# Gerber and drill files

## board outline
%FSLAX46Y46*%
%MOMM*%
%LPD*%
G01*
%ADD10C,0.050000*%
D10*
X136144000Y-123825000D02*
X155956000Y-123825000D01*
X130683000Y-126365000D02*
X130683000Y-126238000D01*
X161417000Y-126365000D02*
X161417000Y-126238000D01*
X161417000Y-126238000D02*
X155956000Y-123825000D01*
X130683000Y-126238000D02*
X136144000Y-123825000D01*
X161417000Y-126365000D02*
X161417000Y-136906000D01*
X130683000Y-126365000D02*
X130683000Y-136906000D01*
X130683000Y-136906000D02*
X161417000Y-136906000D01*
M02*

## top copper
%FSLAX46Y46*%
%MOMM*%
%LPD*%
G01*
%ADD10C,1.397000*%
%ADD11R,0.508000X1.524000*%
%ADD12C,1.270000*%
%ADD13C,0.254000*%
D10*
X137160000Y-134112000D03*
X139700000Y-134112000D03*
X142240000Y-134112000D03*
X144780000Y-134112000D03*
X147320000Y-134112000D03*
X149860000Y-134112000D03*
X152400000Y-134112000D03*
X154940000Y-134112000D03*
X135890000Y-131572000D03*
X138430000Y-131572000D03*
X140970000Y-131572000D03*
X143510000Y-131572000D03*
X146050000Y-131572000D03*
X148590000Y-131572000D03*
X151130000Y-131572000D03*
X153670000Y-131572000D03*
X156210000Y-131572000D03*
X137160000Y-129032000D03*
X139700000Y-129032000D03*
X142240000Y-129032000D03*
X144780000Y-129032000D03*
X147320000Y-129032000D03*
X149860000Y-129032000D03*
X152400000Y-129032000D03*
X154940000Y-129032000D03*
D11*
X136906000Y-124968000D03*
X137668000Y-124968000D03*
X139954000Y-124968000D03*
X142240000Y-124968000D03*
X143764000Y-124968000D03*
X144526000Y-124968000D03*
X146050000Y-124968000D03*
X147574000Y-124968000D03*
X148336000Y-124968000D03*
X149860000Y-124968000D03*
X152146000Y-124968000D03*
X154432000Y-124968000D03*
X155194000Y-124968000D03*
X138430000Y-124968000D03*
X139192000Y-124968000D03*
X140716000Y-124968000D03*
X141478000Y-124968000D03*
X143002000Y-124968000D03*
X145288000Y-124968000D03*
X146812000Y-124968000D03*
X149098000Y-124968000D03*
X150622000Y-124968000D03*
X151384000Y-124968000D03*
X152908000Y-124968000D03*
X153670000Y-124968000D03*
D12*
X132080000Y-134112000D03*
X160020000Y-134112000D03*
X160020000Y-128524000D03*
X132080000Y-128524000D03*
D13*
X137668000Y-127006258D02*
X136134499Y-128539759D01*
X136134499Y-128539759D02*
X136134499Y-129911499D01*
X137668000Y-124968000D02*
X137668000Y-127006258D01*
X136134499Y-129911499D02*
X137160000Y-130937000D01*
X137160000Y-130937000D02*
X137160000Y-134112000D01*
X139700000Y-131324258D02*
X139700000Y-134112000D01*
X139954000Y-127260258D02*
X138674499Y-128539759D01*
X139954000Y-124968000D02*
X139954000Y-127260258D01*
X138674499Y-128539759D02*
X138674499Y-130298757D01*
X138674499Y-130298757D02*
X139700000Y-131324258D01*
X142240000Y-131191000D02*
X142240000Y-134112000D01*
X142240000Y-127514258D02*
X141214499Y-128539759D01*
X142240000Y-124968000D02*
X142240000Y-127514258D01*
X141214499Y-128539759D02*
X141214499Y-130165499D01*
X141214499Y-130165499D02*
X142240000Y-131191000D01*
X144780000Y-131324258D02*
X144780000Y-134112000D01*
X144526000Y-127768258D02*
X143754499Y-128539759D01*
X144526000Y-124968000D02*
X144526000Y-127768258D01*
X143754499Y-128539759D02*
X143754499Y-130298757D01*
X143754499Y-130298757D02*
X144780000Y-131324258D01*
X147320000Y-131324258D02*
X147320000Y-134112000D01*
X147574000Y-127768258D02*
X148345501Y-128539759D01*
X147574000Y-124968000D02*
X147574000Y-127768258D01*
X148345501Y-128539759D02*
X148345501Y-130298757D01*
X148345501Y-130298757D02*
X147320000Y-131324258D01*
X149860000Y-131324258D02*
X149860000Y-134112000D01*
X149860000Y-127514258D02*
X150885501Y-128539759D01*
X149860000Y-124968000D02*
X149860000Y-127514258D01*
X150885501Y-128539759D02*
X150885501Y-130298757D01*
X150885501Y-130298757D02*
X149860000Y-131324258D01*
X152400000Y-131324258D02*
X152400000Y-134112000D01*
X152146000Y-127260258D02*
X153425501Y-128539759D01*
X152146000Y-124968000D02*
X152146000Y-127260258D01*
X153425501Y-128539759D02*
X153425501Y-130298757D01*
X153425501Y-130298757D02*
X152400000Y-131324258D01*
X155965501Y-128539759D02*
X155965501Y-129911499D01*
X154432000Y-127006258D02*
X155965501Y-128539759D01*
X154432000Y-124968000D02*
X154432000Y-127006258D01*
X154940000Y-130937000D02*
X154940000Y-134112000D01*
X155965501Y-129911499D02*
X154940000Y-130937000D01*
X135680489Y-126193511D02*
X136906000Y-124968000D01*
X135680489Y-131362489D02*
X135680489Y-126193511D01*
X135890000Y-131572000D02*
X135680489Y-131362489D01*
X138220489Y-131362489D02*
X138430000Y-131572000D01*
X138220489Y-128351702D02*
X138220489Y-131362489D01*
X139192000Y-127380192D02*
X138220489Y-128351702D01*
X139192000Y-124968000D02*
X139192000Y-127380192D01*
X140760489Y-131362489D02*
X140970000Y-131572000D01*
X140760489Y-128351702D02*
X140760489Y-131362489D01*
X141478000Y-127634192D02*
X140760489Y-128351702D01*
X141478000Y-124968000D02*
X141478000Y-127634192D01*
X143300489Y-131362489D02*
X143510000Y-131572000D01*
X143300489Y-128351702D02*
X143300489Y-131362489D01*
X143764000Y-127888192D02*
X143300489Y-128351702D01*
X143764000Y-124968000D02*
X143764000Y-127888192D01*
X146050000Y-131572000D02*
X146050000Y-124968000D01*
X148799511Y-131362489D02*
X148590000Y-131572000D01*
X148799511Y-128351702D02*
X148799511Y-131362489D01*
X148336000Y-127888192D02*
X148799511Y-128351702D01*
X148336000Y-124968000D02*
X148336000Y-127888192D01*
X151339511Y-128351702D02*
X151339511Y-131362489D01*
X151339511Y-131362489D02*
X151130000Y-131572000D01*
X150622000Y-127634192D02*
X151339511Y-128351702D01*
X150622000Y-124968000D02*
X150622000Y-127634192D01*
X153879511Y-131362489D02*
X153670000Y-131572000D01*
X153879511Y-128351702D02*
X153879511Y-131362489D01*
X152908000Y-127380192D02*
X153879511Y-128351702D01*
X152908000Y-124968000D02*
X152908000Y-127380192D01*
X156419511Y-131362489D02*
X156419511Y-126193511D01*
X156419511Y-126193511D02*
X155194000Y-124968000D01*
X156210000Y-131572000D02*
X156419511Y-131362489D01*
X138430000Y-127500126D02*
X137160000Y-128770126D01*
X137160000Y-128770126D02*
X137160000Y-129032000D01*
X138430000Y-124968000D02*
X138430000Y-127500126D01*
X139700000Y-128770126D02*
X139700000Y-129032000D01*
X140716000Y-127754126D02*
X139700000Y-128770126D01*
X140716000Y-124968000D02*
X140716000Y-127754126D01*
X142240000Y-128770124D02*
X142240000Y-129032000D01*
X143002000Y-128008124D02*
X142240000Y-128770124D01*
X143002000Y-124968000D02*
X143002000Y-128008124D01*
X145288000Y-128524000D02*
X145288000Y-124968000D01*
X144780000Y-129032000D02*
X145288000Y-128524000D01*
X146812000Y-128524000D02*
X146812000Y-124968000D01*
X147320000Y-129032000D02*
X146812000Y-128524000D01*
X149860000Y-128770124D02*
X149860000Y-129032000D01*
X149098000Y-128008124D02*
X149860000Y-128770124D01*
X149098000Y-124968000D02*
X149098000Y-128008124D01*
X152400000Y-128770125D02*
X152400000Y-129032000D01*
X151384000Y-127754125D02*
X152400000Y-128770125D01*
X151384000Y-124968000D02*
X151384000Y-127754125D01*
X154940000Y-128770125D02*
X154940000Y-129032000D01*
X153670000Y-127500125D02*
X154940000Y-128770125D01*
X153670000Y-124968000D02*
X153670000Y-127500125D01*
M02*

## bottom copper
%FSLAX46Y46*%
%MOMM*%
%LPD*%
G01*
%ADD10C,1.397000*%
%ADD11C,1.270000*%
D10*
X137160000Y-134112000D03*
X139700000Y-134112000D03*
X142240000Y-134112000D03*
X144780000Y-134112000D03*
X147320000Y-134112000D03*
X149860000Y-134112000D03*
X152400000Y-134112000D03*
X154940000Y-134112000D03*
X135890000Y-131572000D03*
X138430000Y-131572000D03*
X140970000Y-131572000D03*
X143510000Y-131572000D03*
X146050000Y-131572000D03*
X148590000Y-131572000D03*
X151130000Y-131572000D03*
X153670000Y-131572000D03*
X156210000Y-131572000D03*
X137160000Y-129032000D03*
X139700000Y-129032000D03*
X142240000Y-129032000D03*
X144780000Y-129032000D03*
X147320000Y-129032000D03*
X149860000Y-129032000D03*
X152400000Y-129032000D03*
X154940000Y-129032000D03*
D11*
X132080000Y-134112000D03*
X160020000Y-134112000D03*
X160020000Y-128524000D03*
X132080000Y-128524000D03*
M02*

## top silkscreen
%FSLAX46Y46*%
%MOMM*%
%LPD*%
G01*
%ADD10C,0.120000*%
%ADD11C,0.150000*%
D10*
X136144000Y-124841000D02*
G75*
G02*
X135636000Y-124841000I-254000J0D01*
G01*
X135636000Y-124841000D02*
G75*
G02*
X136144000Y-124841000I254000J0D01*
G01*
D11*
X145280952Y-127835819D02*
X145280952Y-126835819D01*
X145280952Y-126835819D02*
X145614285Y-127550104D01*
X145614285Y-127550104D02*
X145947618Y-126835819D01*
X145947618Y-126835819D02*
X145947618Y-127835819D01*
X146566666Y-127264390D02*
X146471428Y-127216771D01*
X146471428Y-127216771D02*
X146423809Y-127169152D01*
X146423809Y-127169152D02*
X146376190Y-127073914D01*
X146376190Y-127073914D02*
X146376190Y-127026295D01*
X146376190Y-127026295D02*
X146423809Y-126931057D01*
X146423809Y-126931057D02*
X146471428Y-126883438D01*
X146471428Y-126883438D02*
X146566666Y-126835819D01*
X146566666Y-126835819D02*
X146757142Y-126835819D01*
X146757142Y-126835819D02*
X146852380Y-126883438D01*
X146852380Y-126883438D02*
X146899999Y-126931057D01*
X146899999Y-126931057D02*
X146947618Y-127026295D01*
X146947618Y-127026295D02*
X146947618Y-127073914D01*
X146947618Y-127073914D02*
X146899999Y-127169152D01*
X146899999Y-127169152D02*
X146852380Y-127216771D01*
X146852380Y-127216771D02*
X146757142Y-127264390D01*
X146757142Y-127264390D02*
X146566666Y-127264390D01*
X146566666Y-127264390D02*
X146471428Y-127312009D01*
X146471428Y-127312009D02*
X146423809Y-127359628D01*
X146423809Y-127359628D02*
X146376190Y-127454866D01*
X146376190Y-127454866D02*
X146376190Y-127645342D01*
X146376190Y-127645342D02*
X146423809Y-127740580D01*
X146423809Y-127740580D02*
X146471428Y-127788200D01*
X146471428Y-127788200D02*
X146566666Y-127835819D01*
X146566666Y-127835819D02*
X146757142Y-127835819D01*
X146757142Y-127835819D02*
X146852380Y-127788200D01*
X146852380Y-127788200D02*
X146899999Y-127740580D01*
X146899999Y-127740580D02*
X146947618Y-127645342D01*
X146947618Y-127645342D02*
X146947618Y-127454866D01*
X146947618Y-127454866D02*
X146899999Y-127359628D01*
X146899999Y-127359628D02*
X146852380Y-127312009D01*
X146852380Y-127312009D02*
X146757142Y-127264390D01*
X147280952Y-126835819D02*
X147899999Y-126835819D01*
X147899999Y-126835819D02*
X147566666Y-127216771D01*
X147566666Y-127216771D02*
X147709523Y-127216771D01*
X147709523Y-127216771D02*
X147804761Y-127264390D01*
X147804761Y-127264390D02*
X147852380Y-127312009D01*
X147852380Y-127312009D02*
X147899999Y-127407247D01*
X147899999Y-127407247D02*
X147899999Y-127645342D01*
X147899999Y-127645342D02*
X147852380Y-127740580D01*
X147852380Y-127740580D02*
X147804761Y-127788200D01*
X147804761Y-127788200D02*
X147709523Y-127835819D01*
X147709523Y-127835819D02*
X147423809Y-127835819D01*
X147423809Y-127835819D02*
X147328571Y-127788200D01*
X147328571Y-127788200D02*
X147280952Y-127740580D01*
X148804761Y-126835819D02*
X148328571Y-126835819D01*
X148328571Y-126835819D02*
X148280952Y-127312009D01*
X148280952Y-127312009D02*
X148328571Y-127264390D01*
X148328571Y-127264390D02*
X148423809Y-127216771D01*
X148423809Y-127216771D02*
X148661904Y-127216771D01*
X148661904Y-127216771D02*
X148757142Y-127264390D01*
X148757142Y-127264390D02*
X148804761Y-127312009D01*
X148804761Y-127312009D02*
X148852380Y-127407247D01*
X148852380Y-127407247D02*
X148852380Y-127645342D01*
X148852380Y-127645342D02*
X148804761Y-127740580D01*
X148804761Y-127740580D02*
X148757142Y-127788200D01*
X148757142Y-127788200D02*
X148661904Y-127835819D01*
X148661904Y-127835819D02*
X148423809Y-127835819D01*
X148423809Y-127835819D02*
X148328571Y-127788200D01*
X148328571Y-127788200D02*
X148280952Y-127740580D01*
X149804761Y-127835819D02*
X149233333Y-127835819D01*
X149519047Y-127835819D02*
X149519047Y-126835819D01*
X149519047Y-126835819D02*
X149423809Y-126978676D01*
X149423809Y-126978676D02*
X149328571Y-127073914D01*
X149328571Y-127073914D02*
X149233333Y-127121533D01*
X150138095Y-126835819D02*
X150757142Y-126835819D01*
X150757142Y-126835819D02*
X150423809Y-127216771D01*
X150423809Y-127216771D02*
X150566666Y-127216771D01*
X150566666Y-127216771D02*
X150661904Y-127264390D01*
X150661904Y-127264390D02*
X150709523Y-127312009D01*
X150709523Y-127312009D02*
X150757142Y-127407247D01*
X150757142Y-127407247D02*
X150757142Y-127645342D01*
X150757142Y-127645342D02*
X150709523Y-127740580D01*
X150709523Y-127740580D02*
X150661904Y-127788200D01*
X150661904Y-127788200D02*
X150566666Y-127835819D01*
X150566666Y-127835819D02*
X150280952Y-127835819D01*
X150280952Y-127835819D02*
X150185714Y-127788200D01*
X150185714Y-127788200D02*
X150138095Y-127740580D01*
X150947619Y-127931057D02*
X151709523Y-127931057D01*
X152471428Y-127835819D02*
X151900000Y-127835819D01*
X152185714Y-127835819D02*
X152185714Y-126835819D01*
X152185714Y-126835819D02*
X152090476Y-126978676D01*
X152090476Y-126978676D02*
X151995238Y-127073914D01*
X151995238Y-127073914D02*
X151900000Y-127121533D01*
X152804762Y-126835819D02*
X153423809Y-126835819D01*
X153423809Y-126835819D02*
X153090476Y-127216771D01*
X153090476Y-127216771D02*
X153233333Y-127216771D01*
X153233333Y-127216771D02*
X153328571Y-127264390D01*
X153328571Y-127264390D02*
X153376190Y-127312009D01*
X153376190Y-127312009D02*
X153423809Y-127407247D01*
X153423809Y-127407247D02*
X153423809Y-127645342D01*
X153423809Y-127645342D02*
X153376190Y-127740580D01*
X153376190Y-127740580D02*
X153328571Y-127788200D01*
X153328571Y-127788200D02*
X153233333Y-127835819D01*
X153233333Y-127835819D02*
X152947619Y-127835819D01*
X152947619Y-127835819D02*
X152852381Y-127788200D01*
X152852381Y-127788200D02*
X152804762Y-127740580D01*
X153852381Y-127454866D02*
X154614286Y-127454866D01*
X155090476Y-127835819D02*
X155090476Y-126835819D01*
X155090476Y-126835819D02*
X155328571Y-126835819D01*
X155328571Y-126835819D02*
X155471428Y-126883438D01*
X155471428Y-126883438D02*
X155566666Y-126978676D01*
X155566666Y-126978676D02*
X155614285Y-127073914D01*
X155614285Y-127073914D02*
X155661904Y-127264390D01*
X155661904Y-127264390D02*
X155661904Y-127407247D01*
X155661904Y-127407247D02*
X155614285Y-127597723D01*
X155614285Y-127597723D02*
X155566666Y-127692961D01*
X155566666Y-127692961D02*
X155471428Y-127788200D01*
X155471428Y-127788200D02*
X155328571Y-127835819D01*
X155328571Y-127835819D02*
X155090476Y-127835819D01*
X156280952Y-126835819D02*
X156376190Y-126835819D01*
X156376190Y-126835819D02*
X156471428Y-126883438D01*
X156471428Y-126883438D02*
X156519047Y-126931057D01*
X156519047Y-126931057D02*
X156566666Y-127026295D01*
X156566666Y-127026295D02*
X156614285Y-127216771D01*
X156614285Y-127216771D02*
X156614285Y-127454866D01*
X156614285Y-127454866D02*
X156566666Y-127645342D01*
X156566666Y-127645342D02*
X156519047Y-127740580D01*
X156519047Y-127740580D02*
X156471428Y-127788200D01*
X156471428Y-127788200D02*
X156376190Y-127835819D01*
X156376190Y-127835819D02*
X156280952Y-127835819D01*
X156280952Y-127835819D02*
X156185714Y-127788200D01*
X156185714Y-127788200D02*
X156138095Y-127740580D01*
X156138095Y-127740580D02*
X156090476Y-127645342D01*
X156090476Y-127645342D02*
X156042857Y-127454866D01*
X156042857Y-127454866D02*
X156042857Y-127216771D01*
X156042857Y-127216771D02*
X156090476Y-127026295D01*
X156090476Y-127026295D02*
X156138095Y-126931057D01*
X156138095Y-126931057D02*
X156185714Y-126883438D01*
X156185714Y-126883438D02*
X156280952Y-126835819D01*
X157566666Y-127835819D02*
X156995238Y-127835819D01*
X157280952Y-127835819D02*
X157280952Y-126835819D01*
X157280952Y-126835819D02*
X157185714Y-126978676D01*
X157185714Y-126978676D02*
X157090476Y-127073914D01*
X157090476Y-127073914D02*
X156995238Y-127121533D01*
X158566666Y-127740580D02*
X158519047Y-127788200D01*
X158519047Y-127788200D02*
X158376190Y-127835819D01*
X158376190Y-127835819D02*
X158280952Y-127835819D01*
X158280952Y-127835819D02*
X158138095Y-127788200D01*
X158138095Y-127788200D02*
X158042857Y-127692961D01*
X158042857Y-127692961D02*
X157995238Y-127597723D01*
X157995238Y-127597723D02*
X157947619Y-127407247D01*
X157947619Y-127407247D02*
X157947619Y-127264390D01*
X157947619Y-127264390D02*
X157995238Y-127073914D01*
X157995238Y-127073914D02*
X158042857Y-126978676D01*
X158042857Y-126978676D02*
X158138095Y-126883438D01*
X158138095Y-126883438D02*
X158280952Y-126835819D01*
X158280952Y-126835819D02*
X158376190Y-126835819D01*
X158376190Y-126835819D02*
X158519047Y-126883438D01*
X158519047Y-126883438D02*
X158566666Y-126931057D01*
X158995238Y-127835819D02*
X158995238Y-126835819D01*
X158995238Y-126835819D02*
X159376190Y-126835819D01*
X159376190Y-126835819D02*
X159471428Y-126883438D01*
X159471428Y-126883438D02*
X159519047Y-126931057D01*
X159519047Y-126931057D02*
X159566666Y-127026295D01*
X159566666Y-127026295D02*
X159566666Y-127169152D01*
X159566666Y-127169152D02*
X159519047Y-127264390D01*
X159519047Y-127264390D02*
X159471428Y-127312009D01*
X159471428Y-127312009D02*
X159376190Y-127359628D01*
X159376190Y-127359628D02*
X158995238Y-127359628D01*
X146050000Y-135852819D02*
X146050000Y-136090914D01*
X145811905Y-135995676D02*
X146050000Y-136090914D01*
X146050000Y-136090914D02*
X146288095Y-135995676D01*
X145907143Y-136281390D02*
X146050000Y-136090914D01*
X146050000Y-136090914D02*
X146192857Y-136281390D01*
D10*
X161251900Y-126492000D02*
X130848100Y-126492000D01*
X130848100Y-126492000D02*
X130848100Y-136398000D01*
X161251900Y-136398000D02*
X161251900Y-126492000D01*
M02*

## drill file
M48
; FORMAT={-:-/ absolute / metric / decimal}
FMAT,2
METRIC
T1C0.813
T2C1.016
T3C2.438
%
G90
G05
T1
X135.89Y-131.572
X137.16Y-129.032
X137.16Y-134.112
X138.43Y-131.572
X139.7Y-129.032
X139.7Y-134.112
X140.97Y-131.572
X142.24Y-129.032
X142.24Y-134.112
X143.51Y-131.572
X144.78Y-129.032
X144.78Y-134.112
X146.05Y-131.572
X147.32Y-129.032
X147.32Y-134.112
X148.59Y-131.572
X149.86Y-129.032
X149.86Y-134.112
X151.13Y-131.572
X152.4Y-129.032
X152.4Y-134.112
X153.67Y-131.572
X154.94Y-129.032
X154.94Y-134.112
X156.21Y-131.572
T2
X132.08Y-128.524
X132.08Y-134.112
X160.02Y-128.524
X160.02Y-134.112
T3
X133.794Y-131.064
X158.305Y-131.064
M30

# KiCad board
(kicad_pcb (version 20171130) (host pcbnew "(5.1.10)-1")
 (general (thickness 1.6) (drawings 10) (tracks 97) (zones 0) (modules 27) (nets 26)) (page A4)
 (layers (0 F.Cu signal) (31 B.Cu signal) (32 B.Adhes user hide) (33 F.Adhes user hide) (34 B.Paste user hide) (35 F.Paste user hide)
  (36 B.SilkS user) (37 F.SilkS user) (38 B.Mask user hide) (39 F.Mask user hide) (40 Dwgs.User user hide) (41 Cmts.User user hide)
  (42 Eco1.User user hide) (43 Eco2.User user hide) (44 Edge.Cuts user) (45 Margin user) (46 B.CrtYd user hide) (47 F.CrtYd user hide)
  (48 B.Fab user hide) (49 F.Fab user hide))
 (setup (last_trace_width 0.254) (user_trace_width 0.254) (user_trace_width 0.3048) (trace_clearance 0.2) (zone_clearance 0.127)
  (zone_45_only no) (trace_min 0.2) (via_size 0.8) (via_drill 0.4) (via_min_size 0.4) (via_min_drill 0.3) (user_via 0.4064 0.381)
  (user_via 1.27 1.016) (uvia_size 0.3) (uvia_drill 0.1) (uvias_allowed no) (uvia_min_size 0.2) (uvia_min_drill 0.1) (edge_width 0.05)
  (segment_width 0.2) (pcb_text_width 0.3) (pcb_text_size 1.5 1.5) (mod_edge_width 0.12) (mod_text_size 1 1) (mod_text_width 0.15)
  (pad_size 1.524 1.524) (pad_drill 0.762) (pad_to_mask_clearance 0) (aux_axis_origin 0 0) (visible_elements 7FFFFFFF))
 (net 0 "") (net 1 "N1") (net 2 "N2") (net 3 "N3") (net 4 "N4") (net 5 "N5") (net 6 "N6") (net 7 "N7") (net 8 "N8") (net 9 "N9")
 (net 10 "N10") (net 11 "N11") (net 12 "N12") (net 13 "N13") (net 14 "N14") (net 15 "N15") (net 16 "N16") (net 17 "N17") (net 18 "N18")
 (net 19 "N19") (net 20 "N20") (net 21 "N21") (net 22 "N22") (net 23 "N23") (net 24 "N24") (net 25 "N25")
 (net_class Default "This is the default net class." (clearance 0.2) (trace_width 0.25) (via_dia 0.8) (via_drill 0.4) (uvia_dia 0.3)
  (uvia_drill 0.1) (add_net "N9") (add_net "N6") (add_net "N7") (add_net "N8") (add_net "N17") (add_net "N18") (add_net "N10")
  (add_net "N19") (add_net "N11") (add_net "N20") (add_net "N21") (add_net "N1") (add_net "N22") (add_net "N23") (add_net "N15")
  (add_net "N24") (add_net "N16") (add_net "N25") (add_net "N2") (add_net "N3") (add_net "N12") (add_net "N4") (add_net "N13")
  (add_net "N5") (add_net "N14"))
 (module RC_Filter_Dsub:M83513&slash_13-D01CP (layer F.Cu) (at 146.05 137.414 180)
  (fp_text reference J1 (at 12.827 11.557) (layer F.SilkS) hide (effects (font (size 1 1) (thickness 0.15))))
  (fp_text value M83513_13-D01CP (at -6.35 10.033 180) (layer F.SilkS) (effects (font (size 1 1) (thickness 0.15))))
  (fp_line (start -15.2019 10.922) (end 15.2019 10.922) (layer F.SilkS) (width 0.12))
  (fp_line (start 15.2019 10.922) (end 15.2019 1.016) (layer F.SilkS) (width 0.12))
  (fp_line (start -15.2019 1.016) (end -15.2019 10.922) (layer F.SilkS) (width 0.12))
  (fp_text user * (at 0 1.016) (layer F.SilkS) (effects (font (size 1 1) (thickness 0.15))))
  (pad 2 thru_hole circle (at 8.89 3.302 180) (size 1.397 1.397) (drill 0.8128) (layers *.Cu *.Mask) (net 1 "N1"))
  (pad 3 thru_hole circle (at 6.35 3.302 180) (size 1.397 1.397) (drill 0.8128) (layers *.Cu *.Mask) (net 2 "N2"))
  (pad 4 thru_hole circle (at 3.81 3.302 180) (size 1.397 1.397) (drill 0.8128) (layers *.Cu *.Mask) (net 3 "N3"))
  (pad 6 thru_hole circle (at 1.27 3.302 180) (size 1.397 1.397) (drill 0.8128) (layers *.Cu *.Mask) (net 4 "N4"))
  (pad 8 thru_hole circle (at -1.27 3.302 180) (size 1.397 1.397) (drill 0.8128) (layers *.Cu *.Mask) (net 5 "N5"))
  (pad 10 thru_hole circle (at -3.81 3.302 180) (size 1.397 1.397) (drill 0.8128) (layers *.Cu *.Mask) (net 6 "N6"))
  (pad 11 thru_hole circle (at -6.35 3.302 180) (size 1.397 1.397) (drill 0.8128) (layers *.Cu *.Mask) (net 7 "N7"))
  (pad 12 thru_hole circle (at -8.89 3.302 180) (size 1.397 1.397) (drill 0.8128) (layers *.Cu *.Mask) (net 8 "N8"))
  (pad 1 thru_hole circle (at 10.16 5.842 180) (size 1.397 1.397) (drill 0.8128) (layers *.Cu *.Mask) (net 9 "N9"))
  (pad 15 thru_hole circle (at 7.62 5.842 180) (size 1.397 1.397) (drill 0.8128) (layers *.Cu *.Mask) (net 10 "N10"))
  (pad 17 thru_hole circle (at 5.08 5.842 180) (size 1.397 1.397) (drill 0.8128) (layers *.Cu *.Mask) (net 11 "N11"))
  (pad 5 thru_hole circle (at 2.54 5.842 180) (size 1.397 1.397) (drill 0.8128) (layers *.Cu *.Mask) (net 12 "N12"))
  (pad 7 thru_hole circle (at 0 5.842 180) (size 1.397 1.397) (drill 0.8128) (layers *.Cu *.Mask) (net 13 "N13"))
  (pad 9 thru_hole circle (at -2.54 5.842 180) (size 1.397 1.397) (drill 0.8128) (layers *.Cu *.Mask) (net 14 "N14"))
  (pad 22 thru_hole circle (at -5.08 5.842 180) (size 1.397 1.397) (drill 0.8128) (layers *.Cu *.Mask) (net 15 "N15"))
  (pad 24 thru_hole circle (at -7.62 5.842 180) (size 1.397 1.397) (drill 0.8128) (layers *.Cu *.Mask) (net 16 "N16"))
  (pad 13 thru_hole circle (at -10.16 5.842 180) (size 1.397 1.397) (drill 0.8128) (layers *.Cu *.Mask) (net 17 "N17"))
  (pad 14 thru_hole circle (at 8.89 8.382 180) (size 1.397 1.397) (drill 0.8128) (layers *.Cu *.Mask) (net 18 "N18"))
  (pad 16 thru_hole circle (at 6.35 8.382 180) (size 1.397 1.397) (drill 0.8128) (layers *.Cu *.Mask) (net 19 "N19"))
  (pad 18 thru_hole circle (at 3.81 8.382 180) (size 1.397 1.397) (drill 0.8128) (layers *.Cu *.Mask) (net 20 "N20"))
  (pad 19 thru_hole circle (at 1.27 8.382 180) (size 1.397 1.397) (drill 0.8128) (layers *.Cu *.Mask) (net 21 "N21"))
  (pad 20 thru_hole circle (at -1.27 8.382 180) (size 1.397 1.397) (drill 0.8128) (layers *.Cu *.Mask) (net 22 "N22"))
  (pad 21 thru_hole circle (at -3.81 8.382 180) (size 1.397 1.397) (drill 0.8128) (layers *.Cu *.Mask) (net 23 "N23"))
  (pad 23 thru_hole circle (at -6.35 8.382 180) (size 1.397 1.397) (drill 0.8128) (layers *.Cu *.Mask) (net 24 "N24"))
  (pad 25 thru_hole circle (at -8.89 8.382 180) (size 1.397 1.397) (drill 0.8128) (layers *.Cu *.Mask) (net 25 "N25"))
  (pad "" np_thru_hole circle (at -12.2555 6.35 270) (size 2.4384 2.4384) (drill 2.4384) (layers *.Cu *.Mask))
  (pad "" np_thru_hole circle (at 12.2555 6.35 180) (size 2.4384 2.4384) (drill 2.4384) (layers *.Cu *.Mask)))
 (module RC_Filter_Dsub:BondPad (layer F.Cu) (at 136.906 124.968)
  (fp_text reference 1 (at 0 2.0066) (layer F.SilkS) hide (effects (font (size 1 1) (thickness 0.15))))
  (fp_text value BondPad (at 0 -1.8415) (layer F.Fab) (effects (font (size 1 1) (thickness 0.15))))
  (pad 1 smd rect (at 0 0) (size 0.508 1.524) (layers F.Cu F.Paste F.Mask) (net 9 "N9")))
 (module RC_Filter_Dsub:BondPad (layer F.Cu) (at 137.668 124.968)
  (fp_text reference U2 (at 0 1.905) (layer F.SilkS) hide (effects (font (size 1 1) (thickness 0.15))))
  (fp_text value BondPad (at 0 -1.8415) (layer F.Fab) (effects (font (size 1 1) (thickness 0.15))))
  (pad 1 smd rect (at 0 0) (size 0.508 1.524) (layers F.Cu F.Paste F.Mask) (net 1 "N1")))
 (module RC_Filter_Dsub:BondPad (layer F.Cu) (at 139.954 124.968)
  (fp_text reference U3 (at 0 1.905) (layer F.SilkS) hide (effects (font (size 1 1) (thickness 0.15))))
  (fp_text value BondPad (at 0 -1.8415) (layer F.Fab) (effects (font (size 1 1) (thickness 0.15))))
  (pad 1 smd rect (at 0 0) (size 0.508 1.524) (layers F.Cu F.Paste F.Mask) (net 2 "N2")))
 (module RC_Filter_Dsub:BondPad (layer F.Cu) (at 142.24 124.968)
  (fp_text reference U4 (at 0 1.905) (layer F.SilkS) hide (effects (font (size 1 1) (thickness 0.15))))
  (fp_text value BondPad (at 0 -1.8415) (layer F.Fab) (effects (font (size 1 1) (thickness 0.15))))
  (pad 1 smd rect (at 0 0) (size 0.508 1.524) (layers F.Cu F.Paste F.Mask) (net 3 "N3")))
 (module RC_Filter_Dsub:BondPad (layer F.Cu) (at 143.764 124.968)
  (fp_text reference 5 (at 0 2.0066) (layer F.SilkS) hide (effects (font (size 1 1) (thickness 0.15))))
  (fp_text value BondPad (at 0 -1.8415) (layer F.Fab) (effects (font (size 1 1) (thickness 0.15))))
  (pad 1 smd rect (at 0 0) (size 0.508 1.524) (layers F.Cu F.Paste F.Mask) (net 12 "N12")))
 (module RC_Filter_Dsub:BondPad (layer F.Cu) (at 144.526 124.968)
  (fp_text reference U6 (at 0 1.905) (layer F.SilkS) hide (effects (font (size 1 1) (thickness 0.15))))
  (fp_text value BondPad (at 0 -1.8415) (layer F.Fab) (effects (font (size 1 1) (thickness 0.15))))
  (pad 1 smd rect (at 0 0) (size 0.508 1.524) (layers F.Cu F.Paste F.Mask) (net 4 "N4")))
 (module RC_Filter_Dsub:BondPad (layer F.Cu) (at 146.05 124.968)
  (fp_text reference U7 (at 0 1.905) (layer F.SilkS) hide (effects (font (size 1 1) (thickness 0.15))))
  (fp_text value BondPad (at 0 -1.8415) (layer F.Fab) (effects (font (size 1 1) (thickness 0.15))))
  (pad 1 smd rect (at 0 0) (size 0.508 1.524) (layers F.Cu F.Paste F.Mask) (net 13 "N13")))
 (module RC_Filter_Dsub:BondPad (layer F.Cu) (at 147.574 124.968)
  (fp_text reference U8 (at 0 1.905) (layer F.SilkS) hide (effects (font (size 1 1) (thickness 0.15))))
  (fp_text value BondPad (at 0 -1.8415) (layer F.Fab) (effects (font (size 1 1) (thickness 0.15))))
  (pad 1 smd rect (at 0 0) (size 0.508 1.524) (layers F.Cu F.Paste F.Mask) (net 5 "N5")))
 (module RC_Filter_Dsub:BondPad (layer F.Cu) (at 148.336 124.968)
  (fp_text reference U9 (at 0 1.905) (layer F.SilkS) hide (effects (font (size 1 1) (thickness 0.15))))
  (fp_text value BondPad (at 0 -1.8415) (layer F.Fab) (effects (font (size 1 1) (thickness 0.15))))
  (pad 1 smd rect (at 0 0) (size 0.508 1.524) (layers F.Cu F.Paste F.Mask) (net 14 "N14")))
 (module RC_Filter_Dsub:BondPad (layer F.Cu) (at 149.86 124.968)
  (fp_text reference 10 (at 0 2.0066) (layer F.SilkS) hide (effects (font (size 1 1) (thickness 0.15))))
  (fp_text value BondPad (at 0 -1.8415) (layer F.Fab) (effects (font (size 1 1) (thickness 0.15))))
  (pad 1 smd rect (at 0 0) (size 0.508 1.524) (layers F.Cu F.Paste F.Mask) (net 6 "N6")))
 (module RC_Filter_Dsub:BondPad (layer F.Cu) (at 152.146 124.968)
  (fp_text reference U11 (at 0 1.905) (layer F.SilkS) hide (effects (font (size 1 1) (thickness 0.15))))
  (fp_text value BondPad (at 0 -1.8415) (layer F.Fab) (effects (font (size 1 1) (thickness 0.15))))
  (pad 1 smd rect (at 0 0) (size 0.508 1.524) (layers F.Cu F.Paste F.Mask) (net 7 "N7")))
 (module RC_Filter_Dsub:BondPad (layer F.Cu) (at 154.432 124.968)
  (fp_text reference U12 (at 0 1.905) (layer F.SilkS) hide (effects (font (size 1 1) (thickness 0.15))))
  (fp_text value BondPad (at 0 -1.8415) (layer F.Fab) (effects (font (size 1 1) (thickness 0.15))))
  (pad 1 smd rect (at 0 0) (size 0.508 1.524) (layers F.Cu F.Paste F.Mask) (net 8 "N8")))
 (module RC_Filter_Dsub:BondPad (layer F.Cu) (at 155.194 124.968)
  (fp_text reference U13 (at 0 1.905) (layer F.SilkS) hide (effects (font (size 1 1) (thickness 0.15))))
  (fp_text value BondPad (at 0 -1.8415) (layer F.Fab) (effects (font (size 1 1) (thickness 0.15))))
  (pad 1 smd rect (at 0 0) (size 0.508 1.524) (layers F.Cu F.Paste F.Mask) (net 17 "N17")))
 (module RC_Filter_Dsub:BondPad (layer F.Cu) (at 138.43 124.968)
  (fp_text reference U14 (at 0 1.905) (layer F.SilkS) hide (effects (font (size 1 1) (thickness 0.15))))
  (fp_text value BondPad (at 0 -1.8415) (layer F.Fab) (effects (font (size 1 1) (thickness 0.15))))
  (pad 1 smd rect (at 0 0) (size 0.508 1.524) (layers F.Cu F.Paste F.Mask) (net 18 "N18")))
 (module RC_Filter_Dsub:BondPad (layer F.Cu) (at 139.192 124.968)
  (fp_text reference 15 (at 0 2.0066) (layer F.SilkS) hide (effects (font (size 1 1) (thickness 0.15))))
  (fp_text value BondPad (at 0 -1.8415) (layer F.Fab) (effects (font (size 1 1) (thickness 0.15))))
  (pad 1 smd rect (at 0 0) (size 0.508 1.524) (layers F.Cu F.Paste F.Mask) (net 10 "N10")))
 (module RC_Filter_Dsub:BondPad (layer F.Cu) (at 140.716 124.968)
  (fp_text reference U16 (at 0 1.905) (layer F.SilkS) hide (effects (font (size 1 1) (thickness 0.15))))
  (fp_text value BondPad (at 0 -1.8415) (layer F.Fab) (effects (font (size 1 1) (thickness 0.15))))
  (pad 1 smd rect (at 0 0) (size 0.508 1.524) (layers F.Cu F.Paste F.Mask) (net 19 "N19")))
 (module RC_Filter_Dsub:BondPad (layer F.Cu) (at 141.478 124.968)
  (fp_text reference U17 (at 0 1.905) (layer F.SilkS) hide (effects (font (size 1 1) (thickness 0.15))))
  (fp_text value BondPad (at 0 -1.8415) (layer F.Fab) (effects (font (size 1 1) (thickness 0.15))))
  (pad 1 smd rect (at 0 0) (size 0.508 1.524) (layers F.Cu F.Paste F.Mask) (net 11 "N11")))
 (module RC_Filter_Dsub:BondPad (layer F.Cu) (at 143.002 124.968)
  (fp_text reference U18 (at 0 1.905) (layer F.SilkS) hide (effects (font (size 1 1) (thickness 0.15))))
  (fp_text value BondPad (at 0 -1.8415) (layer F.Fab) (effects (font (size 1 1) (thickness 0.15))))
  (pad 1 smd rect (at 0 0) (size 0.508 1.524) (layers F.Cu F.Paste F.Mask) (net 20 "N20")))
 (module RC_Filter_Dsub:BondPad (layer F.Cu) (at 145.288 124.968)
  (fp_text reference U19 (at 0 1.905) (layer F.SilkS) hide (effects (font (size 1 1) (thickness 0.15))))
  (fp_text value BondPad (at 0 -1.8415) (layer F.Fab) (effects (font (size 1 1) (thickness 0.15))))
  (pad 1 smd rect (at 0 0) (size 0.508 1.524) (layers F.Cu F.Paste F.Mask) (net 21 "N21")))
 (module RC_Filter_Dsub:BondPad (layer F.Cu) (at 146.812 124.968)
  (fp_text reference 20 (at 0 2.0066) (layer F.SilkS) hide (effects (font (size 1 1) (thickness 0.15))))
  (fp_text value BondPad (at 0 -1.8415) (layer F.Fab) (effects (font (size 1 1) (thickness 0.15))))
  (pad 1 smd rect (at 0 0) (size 0.508 1.524) (layers F.Cu F.Paste F.Mask) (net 22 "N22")))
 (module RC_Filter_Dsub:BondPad (layer F.Cu) (at 149.098 124.968)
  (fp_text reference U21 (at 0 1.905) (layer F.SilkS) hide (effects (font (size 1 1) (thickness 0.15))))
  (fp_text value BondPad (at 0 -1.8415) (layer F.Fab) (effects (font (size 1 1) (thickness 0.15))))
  (pad 1 smd rect (at 0 0) (size 0.508 1.524) (layers F.Cu F.Paste F.Mask) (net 23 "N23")))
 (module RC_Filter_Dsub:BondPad (layer F.Cu) (at 150.622 124.968)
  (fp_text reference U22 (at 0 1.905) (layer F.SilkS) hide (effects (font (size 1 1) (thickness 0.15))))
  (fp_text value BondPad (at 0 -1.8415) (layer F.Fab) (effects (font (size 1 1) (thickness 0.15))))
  (pad 1 smd rect (at 0 0) (size 0.508 1.524) (layers F.Cu F.Paste F.Mask) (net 15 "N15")))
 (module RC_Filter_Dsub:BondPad (layer F.Cu) (at 151.384 124.968)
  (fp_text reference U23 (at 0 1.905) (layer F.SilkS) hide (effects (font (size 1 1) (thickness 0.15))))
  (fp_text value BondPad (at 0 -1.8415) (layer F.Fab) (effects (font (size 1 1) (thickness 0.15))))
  (pad 1 smd rect (at 0 0) (size 0.508 1.524) (layers F.Cu F.Paste F.Mask) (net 24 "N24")))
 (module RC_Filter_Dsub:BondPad (layer F.Cu) (at 152.908 124.968)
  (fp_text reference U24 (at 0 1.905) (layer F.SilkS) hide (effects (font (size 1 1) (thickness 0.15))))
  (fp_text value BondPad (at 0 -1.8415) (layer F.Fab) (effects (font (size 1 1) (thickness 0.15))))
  (pad 1 smd rect (at 0 0) (size 0.508 1.524) (layers F.Cu F.Paste F.Mask) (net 16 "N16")))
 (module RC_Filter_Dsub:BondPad (layer F.Cu) (at 153.67 124.968)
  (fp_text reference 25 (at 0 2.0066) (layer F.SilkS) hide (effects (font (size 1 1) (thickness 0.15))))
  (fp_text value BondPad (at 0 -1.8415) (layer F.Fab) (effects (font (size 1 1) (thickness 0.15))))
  (pad 1 smd rect (at 0 0) (size 0.508 1.524) (layers F.Cu F.Paste F.Mask) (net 25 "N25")))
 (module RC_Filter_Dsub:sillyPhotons (layer F.Cu) (at 134.366 134.366)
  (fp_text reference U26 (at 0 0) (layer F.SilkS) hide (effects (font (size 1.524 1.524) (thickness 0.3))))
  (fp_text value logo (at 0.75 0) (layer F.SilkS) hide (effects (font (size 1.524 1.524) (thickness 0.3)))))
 (gr_circle (center 135.89 124.841) (end 135.89 124.587) (layer F.SilkS) (width 0.12))
 (gr_line (start 136.144 123.825) (end 155.956 123.825) (layer Edge.Cuts) (width 0.05))
 (gr_line (start 130.683 126.365) (end 130.683 126.238) (layer Edge.Cuts) (width 0.05))
 (gr_line (start 161.417 126.365) (end 161.417 126.238) (layer Edge.Cuts) (width 0.05))
 (gr_line (start 161.417 126.238) (end 155.956 123.825) (layer Edge.Cuts) (width 0.05))
 (gr_line (start 130.683 126.238) (end 136.144 123.825) (layer Edge.Cuts) (width 0.05))
 (gr_line (start 161.417 126.365) (end 161.417 136.906) (layer Edge.Cuts) (width 0.05))
 (gr_line (start 130.683 126.365) (end 130.683 136.906) (layer Edge.Cuts) (width 0.05))
 (gr_line (start 130.683 136.906) (end 161.417 136.906) (layer Edge.Cuts) (width 0.05))
 (via (at 132.08 134.112) (size 1.27) (drill 1.016) (layers F.Cu B.Cu) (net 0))
 (via (at 160.02 134.112) (size 1.27) (drill 1.016) (layers F.Cu B.Cu) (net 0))
 (via (at 160.02 128.524) (size 1.27) (drill 1.016) (layers F.Cu B.Cu) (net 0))
 (via (at 132.08 128.524) (size 1.27) (drill 1.016) (layers F.Cu B.Cu) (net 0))
 (segment (start 137.668 127.006258) (end 136.134499 128.539759) (width 0.254) (layer F.Cu) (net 1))
 (segment (start 136.134499 128.539759) (end 136.134499 129.911499) (width 0.254) (layer F.Cu) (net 1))
 (segment (start 137.668 124.968) (end 137.668 127.006258) (width 0.254) (layer F.Cu) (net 1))
 (segment (start 136.134499 129.911499) (end 137.16 130.937) (width 0.254) (layer F.Cu) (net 1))
 (segment (start 137.16 130.937) (end 137.16 134.112) (width 0.254) (layer F.Cu) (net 1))
 (segment (start 139.7 131.324258) (end 139.7 134.112) (width 0.254) (layer F.Cu) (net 2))
 (segment (start 139.954 127.260258) (end 138.674499 128.539759) (width 0.254) (layer F.Cu) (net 2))
 (segment (start 139.954 124.968) (end 139.954 127.260258) (width 0.254) (layer F.Cu) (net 2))
 (segment (start 138.674499 128.539759) (end 138.674499 130.298757) (width 0.254) (layer F.Cu) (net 2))
 (segment (start 138.674499 130.298757) (end 139.7 131.324258) (width 0.254) (layer F.Cu) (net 2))
 (segment (start 142.24 131.191) (end 142.24 134.112) (width 0.254) (layer F.Cu) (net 3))
 (segment (start 142.24 127.514258) (end 141.214499 128.539759) (width 0.254) (layer F.Cu) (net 3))
 (segment (start 142.24 124.968) (end 142.24 127.514258) (width 0.254) (layer F.Cu) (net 3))
 (segment (start 141.214499 128.539759) (end 141.214499 130.165499) (width 0.254) (layer F.Cu) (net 3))
 (segment (start 141.214499 130.165499) (end 142.24 131.191) (width 0.254) (layer F.Cu) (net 3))
 (segment (start 144.78 131.324258) (end 144.78 134.112) (width 0.254) (layer F.Cu) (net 4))
 (segment (start 144.526 127.768258) (end 143.754499 128.539759) (width 0.254) (layer F.Cu) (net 4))
 (segment (start 144.526 124.968) (end 144.526 127.768258) (width 0.254) (layer F.Cu) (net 4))
 (segment (start 143.754499 128.539759) (end 143.754499 130.298757) (width 0.254) (layer F.Cu) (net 4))
 (segment (start 143.754499 130.298757) (end 144.78 131.324258) (width 0.254) (layer F.Cu) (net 4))
 (segment (start 147.32 131.324258) (end 147.32 134.112) (width 0.254) (layer F.Cu) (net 5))
 (segment (start 147.574 127.768258) (end 148.345501 128.539759) (width 0.254) (layer F.Cu) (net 5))
 (segment (start 147.574 124.968) (end 147.574 127.768258) (width 0.254) (layer F.Cu) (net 5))
 (segment (start 148.345501 128.539759) (end 148.345501 130.298757) (width 0.254) (layer F.Cu) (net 5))
 (segment (start 148.345501 130.298757) (end 147.32 131.324258) (width 0.254) (layer F.Cu) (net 5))
 (segment (start 149.86 131.324258) (end 149.86 134.112) (width 0.254) (layer F.Cu) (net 6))
 (segment (start 149.86 127.514258) (end 150.885501 128.539759) (width 0.254) (layer F.Cu) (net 6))
 (segment (start 149.86 124.968) (end 149.86 127.514258) (width 0.254) (layer F.Cu) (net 6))
 (segment (start 150.885501 128.539759) (end 150.885501 130.298757) (width 0.254) (layer F.Cu) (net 6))
 (segment (start 150.885501 130.298757) (end 149.86 131.324258) (width 0.254) (layer F.Cu) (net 6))
 (segment (start 152.4 131.324258) (end 152.4 134.112) (width 0.254) (layer F.Cu) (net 7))
 (segment (start 152.146 127.260258) (end 153.425501 128.539759) (width 0.254) (layer F.Cu) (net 7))
 (segment (start 152.146 124.968) (end 152.146 127.260258) (width 0.254) (layer F.Cu) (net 7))
 (segment (start 153.425501 128.539759) (end 153.425501 130.298757) (width 0.254) (layer F.Cu) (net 7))
 (segment (start 153.425501 130.298757) (end 152.4 131.324258) (width 0.254) (layer F.Cu) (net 7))
 (segment (start 155.965501 128.539759) (end 155.965501 129.911499) (width 0.254) (layer F.Cu) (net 8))
 (segment (start 154.432 127.006258) (end 155.965501 128.539759) (width 0.254) (layer F.Cu) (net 8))
 (segment (start 154.432 124.968) (end 154.432 127.006258) (width 0.254) (layer F.Cu) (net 8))
 (segment (start 154.94 130.937) (end 154.94 134.112) (width 0.254) (layer F.Cu) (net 8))
 (segment (start 155.965501 129.911499) (end 154.94 130.937) (width 0.254) (layer F.Cu) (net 8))
 (segment (start 135.680489 126.193511) (end 136.906 124.968) (width 0.254) (layer F.Cu) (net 9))
 (segment (start 135.680489 131.362489) (end 135.680489 126.193511) (width 0.254) (layer F.Cu) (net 9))
 (segment (start 135.89 131.572) (end 135.680489 131.362489) (width 0.254) (layer F.Cu) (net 9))
 (segment (start 138.220489 131.362489) (end 138.43 131.572) (width 0.254) (layer F.Cu) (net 10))
 (segment (start 138.220489 128.351702) (end 138.220489 131.362489) (width 0.254) (layer F.Cu) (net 10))
 (segment (start 139.192 127.380192) (end 138.220489 128.351702) (width 0.254) (layer F.Cu) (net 10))
 (segment (start 139.192 124.968) (end 139.192 127.380192) (width 0.254) (layer F.Cu) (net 10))
 (segment (start 140.760489 131.362489) (end 140.97 131.572) (width 0.254) (layer F.Cu) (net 11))
 (segment (start 140.760489 128.351702) (end 140.760489 131.362489) (width 0.254) (layer F.Cu) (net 11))
 (segment (start 141.478 127.634192) (end 140.760489 128.351702) (width 0.254) (layer F.Cu) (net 11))
 (segment (start 141.478 124.968) (end 141.478 127.634192) (width 0.254) (layer F.Cu) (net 11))
 (segment (start 143.300489 131.362489) (end 143.51 131.572) (width 0.254) (layer F.Cu) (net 12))
 (segment (start 143.300489 128.351702) (end 143.300489 131.362489) (width 0.254) (layer F.Cu) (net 12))
 (segment (start 143.764 127.888192) (end 143.300489 128.351702) (width 0.254) (layer F.Cu) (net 12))
 (segment (start 143.764 124.968) (end 143.764 127.888192) (width 0.254) (layer F.Cu) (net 12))
 (segment (start 146.05 131.572) (end 146.05 124.968) (width 0.254) (layer F.Cu) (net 13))
 (segment (start 148.799511 131.362489) (end 148.59 131.572) (width 0.254) (layer F.Cu) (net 14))
 (segment (start 148.799511 128.351702) (end 148.799511 131.362489) (width 0.254) (layer F.Cu) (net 14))
 (segment (start 148.336 127.888192) (end 148.799511 128.351702) (width 0.254) (layer F.Cu) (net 14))
 (segment (start 148.336 124.968) (end 148.336 127.888192) (width 0.254) (layer F.Cu) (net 14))
 (segment (start 151.339511 128.351702) (end 151.339511 131.362489) (width 0.254) (layer F.Cu) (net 15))
 (segment (start 151.339511 131.362489) (end 151.13 131.572) (width 0.254) (layer F.Cu) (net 15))
 (segment (start 150.622 127.634192) (end 151.339511 128.351702) (width 0.254) (layer F.Cu) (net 15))
 (segment (start 150.622 124.968) (end 150.622 127.634192) (width 0.254) (layer F.Cu) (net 15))
 (segment (start 153.879511 131.362489) (end 153.67 131.572) (width 0.254) (layer F.Cu) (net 16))
 (segment (start 153.879511 128.351702) (end 153.879511 131.362489) (width 0.254) (layer F.Cu) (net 16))
 (segment (start 152.908 127.380192) (end 153.879511 128.351702) (width 0.254) (layer F.Cu) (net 16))
 (segment (start 152.908 124.968) (end 152.908 127.380192) (width 0.254) (layer F.Cu) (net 16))
 (segment (start 156.419511 131.362489) (end 156.419511 126.193511) (width 0.254) (layer F.Cu) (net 17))
 (segment (start 156.419511 126.193511) (end 155.194 124.968) (width 0.254) (layer F.Cu) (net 17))
 (segment (start 156.21 131.572) (end 156.419511 131.362489) (width 0.254) (layer F.Cu) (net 17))
 (segment (start 138.43 127.500126) (end 137.16 128.770126) (width 0.254) (layer F.Cu) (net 18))
 (segment (start 137.16 128.770126) (end 137.16 129.032) (width 0.254) (layer F.Cu) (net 18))
 (segment (start 138.43 124.968) (end 138.43 127.500126) (width 0.254) (layer F.Cu) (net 18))
 (segment (start 139.7 128.770126) (end 139.7 129.032) (width 0.254) (layer F.Cu) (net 19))
 (segment (start 140.716 127.754126) (end 139.7 128.770126) (width 0.254) (layer F.Cu) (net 19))
 (segment (start 140.716 124.968) (end 140.716 127.754126) (width 0.254) (layer F.Cu) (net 19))
 (segment (start 142.24 128.770124) (end 142.24 129.032) (width 0.254) (layer F.Cu) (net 20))
 (segment (start 143.002 128.008124) (end 142.24 128.770124) (width 0.254) (layer F.Cu) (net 20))
 (segment (start 143.002 124.968) (end 143.002 128.008124) (width 0.254) (layer F.Cu) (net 20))
 (segment (start 145.288 128.524) (end 145.288 124.968) (width 0.254) (layer F.Cu) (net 21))
 (segment (start 144.78 129.032) (end 145.288 128.524) (width 0.254) (layer F.Cu) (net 21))
 (segment (start 146.812 128.524) (end 146.812 124.968) (width 0.254) (layer F.Cu) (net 22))
 (segment (start 147.32 129.032) (end 146.812 128.524) (width 0.254) (layer F.Cu) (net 22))
 (segment (start 149.86 128.770124) (end 149.86 129.032) (width 0.254) (layer F.Cu) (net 23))
 (segment (start 149.098 128.008124) (end 149.86 128.770124) (width 0.254) (layer F.Cu) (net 23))
 (segment (start 149.098 124.968) (end 149.098 128.008124) (width 0.254) (layer F.Cu) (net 23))
 (segment (start 152.4 128.770125) (end 152.4 129.032) (width 0.254) (layer F.Cu) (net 24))
 (segment (start 151.384 127.754125) (end 152.4 128.770125) (width 0.254) (layer F.Cu) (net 24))
 (segment (start 151.384 124.968) (end 151.384 127.754125) (width 0.254) (layer F.Cu) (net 24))
 (segment (start 154.94 128.770125) (end 154.94 129.032) (width 0.254) (layer F.Cu) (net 25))
 (segment (start 153.67 127.500125) (end 154.94 128.770125) (width 0.254) (layer F.Cu) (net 25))
 (segment (start 153.67 124.968) (end 153.67 127.500125) (width 0.254) (layer F.Cu) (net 25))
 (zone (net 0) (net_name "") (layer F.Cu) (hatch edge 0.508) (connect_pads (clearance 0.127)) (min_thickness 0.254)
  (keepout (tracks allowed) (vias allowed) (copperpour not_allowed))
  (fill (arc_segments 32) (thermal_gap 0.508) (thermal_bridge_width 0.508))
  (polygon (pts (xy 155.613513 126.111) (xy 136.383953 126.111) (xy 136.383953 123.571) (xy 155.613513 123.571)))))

